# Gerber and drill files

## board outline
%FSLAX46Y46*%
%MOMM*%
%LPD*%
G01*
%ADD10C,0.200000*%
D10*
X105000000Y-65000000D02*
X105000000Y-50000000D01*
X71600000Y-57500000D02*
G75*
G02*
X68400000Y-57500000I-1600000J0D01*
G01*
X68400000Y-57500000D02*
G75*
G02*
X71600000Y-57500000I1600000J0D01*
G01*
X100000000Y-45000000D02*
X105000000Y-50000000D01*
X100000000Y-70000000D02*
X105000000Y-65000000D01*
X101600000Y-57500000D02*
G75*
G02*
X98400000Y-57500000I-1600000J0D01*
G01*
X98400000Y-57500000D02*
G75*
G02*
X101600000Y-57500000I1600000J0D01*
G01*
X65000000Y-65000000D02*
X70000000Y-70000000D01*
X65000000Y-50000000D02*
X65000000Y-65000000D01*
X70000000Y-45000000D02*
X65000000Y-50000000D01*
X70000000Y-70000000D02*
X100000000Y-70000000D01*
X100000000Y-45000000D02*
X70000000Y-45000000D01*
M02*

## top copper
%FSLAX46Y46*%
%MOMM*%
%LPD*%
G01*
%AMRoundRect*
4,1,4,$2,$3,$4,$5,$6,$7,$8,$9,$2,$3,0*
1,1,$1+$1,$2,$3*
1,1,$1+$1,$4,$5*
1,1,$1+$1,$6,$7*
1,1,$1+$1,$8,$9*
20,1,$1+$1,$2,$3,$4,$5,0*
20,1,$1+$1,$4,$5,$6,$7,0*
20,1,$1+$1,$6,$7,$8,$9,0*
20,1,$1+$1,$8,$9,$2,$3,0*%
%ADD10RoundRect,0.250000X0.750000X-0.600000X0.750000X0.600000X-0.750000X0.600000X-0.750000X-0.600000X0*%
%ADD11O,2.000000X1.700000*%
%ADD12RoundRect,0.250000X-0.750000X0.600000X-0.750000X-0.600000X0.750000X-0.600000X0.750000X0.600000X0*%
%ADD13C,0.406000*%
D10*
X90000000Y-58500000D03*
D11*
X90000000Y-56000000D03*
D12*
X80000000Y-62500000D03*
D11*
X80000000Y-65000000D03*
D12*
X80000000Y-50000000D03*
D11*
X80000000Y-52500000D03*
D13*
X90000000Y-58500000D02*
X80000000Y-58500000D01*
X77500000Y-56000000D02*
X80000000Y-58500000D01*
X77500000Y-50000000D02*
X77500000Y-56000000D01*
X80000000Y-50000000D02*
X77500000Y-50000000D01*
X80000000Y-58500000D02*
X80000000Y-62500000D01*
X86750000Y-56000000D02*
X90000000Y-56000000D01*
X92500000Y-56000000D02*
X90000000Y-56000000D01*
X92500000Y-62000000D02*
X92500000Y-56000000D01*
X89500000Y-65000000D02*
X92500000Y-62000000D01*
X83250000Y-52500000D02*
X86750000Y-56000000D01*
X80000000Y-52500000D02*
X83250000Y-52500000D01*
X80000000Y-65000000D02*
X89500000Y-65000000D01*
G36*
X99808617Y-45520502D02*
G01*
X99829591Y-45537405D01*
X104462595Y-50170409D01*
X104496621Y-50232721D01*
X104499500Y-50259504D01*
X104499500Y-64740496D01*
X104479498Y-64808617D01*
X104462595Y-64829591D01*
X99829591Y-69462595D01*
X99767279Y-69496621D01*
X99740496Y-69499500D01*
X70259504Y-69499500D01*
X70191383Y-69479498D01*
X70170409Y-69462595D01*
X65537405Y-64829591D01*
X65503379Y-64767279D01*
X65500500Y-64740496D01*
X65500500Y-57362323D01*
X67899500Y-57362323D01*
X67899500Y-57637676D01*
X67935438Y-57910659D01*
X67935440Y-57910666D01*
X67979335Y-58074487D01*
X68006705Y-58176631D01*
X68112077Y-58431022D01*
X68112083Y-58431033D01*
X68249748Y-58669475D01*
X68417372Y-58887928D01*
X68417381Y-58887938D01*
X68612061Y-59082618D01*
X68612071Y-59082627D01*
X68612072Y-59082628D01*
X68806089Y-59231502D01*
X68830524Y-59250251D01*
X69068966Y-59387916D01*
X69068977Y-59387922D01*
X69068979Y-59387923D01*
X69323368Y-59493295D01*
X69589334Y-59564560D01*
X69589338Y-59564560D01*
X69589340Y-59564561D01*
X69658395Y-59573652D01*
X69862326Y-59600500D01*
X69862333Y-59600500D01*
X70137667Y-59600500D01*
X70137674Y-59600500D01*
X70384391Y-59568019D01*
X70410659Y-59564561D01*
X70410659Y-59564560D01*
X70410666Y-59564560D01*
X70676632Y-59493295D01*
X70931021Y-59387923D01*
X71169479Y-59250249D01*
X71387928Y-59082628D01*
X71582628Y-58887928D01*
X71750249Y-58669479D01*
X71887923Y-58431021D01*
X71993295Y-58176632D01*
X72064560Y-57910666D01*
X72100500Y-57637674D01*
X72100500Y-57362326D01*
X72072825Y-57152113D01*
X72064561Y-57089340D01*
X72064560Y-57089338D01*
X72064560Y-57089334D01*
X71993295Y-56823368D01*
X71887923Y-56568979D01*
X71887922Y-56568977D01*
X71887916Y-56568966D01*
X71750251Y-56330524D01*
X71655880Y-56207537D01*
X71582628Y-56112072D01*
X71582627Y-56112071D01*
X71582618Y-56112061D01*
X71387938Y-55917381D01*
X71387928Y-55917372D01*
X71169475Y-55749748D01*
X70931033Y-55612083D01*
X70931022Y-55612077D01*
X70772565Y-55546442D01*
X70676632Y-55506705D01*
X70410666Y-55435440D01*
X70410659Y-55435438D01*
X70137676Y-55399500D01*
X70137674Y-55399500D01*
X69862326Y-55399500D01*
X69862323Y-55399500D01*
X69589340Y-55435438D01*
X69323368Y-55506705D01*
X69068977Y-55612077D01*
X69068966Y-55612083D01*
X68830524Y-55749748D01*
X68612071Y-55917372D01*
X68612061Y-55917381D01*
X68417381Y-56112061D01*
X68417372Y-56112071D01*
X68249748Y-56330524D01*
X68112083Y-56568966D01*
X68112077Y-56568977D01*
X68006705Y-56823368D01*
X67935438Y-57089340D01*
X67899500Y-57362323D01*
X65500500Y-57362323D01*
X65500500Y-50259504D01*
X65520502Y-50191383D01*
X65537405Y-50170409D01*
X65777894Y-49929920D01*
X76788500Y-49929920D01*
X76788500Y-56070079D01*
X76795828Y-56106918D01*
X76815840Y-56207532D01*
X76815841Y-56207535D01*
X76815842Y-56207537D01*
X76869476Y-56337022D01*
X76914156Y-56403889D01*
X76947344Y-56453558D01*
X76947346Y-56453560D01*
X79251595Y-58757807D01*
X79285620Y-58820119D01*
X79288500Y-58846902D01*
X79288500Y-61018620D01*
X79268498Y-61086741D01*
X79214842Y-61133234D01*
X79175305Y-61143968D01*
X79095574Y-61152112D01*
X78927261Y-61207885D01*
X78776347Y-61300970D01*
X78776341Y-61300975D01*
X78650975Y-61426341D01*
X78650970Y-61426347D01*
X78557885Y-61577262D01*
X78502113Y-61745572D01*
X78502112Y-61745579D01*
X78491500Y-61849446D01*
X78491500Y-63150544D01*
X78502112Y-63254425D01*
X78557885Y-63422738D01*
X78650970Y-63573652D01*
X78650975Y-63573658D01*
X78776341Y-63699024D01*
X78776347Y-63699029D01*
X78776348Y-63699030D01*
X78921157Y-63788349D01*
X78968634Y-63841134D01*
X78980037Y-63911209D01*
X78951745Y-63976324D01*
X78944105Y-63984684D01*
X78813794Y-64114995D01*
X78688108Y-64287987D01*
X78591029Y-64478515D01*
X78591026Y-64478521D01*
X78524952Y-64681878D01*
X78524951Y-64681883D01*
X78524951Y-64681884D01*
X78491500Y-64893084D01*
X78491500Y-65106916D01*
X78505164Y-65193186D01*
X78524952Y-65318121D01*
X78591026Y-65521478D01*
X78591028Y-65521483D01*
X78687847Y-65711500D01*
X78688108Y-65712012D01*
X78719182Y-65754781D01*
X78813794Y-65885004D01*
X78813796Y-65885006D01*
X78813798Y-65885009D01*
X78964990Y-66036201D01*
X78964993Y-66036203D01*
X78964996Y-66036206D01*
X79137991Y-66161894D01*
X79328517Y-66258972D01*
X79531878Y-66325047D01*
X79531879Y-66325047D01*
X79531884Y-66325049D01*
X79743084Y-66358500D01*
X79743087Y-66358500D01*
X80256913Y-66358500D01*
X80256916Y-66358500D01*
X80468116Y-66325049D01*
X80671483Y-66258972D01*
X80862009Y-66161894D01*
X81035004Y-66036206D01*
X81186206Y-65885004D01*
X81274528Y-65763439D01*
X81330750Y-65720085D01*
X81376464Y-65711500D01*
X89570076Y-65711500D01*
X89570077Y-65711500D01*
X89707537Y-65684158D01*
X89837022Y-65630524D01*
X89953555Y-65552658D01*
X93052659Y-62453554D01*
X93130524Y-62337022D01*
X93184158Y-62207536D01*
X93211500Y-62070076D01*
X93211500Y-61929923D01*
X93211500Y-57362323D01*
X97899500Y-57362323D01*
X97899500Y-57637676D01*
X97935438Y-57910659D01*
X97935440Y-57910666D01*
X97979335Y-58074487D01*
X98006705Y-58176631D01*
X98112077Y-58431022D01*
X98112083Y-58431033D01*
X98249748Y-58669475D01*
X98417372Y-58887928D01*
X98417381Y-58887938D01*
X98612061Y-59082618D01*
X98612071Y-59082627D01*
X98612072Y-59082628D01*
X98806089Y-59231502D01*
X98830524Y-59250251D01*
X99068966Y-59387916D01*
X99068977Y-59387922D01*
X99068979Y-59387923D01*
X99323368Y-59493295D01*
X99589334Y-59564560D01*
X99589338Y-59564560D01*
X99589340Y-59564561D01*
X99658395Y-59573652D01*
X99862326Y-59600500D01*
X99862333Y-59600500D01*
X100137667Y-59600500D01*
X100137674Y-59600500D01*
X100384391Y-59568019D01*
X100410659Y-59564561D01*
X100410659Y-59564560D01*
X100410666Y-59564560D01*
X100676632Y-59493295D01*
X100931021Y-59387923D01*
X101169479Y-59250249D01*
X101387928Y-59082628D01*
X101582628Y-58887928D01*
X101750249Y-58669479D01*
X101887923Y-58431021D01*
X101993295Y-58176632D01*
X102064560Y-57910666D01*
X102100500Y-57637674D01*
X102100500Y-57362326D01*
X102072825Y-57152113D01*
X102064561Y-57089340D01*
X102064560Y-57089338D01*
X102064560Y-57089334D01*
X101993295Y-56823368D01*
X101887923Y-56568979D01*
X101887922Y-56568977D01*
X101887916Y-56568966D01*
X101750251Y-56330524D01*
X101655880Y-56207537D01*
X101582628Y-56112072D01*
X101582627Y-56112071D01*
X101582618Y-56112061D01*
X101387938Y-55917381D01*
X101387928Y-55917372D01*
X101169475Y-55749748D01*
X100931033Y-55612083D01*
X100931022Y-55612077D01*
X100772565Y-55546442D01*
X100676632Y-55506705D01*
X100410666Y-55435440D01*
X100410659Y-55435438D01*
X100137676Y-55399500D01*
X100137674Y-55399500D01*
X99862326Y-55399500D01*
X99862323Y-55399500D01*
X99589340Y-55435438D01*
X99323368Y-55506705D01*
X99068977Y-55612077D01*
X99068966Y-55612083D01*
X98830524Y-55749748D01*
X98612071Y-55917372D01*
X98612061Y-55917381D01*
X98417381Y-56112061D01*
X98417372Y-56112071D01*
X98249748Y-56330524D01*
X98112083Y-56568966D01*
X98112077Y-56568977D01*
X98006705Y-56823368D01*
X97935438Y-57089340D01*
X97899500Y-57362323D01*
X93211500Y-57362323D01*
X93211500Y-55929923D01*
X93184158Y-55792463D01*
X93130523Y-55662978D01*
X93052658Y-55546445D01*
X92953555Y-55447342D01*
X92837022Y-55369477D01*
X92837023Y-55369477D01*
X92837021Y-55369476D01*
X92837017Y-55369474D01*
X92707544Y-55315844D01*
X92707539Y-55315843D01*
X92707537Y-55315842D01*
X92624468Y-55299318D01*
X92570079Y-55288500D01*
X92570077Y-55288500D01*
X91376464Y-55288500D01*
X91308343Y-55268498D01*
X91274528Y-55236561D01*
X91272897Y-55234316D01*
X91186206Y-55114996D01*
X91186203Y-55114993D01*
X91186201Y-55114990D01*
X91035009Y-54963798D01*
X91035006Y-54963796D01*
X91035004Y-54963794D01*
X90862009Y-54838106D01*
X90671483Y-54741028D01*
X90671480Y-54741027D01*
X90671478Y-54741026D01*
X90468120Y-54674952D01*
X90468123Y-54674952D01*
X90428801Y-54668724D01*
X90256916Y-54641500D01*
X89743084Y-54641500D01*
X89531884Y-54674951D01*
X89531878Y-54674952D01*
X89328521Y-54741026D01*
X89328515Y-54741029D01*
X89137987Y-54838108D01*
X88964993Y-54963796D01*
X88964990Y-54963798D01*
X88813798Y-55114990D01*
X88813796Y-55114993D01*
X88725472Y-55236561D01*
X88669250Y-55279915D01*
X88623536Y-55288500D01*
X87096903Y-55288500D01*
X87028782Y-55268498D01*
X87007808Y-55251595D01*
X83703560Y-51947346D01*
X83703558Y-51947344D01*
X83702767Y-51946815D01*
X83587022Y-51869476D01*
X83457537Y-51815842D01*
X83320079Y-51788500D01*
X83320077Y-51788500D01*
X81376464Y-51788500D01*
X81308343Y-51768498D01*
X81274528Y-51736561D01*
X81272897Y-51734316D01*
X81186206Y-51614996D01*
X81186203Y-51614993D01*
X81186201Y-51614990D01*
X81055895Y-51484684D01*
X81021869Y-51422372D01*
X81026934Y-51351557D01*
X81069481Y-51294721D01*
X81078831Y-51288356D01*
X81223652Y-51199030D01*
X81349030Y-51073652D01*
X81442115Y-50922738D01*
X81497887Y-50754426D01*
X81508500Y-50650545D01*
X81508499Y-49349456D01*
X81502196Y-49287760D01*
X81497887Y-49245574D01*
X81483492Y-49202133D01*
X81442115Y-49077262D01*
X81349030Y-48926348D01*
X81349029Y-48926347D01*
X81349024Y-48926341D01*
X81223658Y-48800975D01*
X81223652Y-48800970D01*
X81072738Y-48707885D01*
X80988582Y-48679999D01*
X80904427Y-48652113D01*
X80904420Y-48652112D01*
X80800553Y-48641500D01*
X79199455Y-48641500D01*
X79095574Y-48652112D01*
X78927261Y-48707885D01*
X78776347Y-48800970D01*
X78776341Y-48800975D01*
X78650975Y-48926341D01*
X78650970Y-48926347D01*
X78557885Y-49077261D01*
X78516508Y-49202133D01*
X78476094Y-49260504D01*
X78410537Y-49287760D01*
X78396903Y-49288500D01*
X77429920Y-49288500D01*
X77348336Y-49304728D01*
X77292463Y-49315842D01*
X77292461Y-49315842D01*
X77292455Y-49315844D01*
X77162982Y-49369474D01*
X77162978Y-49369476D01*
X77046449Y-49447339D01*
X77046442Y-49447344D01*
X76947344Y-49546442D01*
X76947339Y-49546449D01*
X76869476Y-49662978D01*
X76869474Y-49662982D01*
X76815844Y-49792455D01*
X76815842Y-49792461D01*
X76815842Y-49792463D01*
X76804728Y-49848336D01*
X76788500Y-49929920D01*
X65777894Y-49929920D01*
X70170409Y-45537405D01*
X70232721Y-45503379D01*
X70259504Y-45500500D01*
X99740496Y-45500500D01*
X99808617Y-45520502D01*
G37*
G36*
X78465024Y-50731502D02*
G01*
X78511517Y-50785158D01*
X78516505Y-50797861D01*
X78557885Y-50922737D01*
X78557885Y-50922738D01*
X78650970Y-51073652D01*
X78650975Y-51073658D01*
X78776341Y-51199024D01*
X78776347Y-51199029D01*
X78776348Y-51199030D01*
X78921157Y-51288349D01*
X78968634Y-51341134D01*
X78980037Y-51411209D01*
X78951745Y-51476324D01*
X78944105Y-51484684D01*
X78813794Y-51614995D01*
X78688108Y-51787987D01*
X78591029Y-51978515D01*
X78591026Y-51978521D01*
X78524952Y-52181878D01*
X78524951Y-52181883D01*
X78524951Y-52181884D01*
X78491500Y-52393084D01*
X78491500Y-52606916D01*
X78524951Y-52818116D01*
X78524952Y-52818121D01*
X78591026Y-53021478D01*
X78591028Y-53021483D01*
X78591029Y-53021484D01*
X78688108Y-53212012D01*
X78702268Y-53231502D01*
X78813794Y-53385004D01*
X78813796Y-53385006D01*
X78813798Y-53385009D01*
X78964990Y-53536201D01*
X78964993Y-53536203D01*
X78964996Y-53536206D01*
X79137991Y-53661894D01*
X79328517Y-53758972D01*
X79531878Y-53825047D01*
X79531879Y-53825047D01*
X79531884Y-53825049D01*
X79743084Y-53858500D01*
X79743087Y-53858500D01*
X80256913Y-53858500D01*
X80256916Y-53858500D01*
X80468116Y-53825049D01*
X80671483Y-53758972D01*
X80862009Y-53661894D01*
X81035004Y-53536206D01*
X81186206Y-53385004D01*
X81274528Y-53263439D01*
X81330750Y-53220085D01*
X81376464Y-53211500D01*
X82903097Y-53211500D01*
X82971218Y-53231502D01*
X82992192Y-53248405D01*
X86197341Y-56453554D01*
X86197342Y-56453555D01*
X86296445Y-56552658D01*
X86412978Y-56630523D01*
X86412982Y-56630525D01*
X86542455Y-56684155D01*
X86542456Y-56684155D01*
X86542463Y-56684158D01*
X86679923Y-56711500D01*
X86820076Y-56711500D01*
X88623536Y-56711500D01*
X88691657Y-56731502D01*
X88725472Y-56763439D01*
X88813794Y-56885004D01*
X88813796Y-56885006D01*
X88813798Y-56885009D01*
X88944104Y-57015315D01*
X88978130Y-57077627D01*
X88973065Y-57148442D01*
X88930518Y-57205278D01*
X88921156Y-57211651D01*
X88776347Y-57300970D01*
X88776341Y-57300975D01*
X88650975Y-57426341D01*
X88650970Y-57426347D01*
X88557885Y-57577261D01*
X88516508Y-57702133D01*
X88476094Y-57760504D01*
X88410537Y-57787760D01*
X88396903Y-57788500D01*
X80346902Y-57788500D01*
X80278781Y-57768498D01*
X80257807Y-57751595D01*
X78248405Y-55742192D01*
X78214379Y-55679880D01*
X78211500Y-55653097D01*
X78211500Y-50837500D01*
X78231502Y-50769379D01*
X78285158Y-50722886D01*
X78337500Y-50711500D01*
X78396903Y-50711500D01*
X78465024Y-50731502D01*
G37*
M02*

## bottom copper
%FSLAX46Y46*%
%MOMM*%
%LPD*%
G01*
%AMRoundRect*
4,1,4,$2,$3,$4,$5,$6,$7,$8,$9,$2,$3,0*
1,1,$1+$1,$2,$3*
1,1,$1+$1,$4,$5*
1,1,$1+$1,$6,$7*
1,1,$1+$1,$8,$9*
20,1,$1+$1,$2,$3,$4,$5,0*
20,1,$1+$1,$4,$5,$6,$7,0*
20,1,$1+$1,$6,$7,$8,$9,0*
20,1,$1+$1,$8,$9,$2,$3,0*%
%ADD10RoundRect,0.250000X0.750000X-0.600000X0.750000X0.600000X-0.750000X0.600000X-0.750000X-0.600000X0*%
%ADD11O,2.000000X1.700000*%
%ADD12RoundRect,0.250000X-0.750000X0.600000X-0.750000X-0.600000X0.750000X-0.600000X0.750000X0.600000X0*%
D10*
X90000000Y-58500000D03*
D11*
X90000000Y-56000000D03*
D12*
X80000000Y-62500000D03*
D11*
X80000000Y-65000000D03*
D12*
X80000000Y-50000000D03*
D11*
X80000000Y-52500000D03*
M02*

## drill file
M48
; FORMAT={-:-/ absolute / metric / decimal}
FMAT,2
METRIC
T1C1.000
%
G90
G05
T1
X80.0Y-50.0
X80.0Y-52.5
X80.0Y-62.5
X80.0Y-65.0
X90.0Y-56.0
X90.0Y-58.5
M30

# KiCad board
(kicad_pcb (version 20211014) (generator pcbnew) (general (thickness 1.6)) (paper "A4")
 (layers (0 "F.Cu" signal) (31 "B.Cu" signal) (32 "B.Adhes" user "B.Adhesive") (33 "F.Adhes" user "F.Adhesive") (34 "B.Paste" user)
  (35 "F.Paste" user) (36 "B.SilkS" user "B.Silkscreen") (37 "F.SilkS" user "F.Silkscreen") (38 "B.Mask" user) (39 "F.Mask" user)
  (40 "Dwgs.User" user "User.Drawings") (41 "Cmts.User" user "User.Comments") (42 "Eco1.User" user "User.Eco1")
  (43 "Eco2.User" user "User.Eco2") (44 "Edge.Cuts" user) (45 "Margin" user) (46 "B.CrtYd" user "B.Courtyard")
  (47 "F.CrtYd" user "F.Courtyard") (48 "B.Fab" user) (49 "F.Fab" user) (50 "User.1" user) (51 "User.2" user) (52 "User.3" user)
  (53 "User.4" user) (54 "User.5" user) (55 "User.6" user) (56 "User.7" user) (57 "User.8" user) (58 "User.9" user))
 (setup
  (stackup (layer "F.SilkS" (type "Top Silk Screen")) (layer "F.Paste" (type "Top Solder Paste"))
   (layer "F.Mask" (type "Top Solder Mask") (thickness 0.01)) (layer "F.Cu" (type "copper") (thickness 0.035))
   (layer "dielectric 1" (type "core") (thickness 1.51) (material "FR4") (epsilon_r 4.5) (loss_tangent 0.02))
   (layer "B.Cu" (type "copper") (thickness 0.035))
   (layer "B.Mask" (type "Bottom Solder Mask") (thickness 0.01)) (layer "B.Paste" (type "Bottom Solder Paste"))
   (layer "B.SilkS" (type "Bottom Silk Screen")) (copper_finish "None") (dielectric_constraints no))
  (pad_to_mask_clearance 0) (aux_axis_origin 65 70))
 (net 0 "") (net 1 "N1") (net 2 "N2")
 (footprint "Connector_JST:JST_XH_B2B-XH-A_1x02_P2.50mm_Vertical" (layer "F.Cu") (at 90 58.5 90)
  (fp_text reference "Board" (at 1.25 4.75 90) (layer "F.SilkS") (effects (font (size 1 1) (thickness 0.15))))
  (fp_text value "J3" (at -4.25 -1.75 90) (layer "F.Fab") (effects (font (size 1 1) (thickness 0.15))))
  (pad "1" thru_hole roundrect (at 0 0 90) (size 1.7 2) (drill 1) (layers *.Cu *.Mask) (roundrect_rratio 0.1470588235) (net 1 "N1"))
  (pad "2" thru_hole oval (at 2.5 0 90) (size 1.7 2) (drill 1) (layers *.Cu *.Mask) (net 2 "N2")))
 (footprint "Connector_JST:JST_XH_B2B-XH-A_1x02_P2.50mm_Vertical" (layer "F.Cu") (at 80 62.5 -90)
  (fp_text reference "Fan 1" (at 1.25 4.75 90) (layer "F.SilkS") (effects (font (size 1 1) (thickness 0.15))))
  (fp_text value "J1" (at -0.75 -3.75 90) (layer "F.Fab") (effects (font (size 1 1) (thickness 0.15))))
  (pad "1" thru_hole roundrect (at 0 0 270) (size 1.7 2) (drill 1) (layers *.Cu *.Mask) (roundrect_rratio 0.1470588235) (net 1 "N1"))
  (pad "2" thru_hole oval (at 2.5 0 270) (size 1.7 2) (drill 1) (layers *.Cu *.Mask) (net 2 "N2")))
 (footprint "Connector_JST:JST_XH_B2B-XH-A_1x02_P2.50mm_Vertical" (layer "F.Cu") (at 80 50 -90)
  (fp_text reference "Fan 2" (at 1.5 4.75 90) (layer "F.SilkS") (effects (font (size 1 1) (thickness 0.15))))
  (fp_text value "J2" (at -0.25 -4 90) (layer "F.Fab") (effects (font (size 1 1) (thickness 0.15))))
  (pad "1" thru_hole roundrect (at 0 0 270) (size 1.7 2) (drill 1) (layers *.Cu *.Mask) (roundrect_rratio 0.1470588235) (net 1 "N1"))
  (pad "2" thru_hole oval (at 2.5 0 270) (size 1.7 2) (drill 1) (layers *.Cu *.Mask) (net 2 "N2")))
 (gr_line (start 105 65) (end 105 50) (layer "Edge.Cuts") (width 0.2))
 (gr_circle (center 70 57.5) (end 71.6 57.5) (layer "Edge.Cuts") (width 0.2) (fill none))
 (gr_line (start 100 45) (end 105 50) (layer "Edge.Cuts") (width 0.2))
 (gr_line (start 100 70) (end 105 65) (layer "Edge.Cuts") (width 0.2))
 (gr_circle (center 100 57.5) (end 101.6 57.5) (layer "Edge.Cuts") (width 0.2) (fill none))
 (gr_line (start 65 65) (end 70 70) (layer "Edge.Cuts") (width 0.2))
 (gr_line (start 65 50) (end 65 65) (layer "Edge.Cuts") (width 0.2))
 (gr_line (start 70 45) (end 65 50) (layer "Edge.Cuts") (width 0.2))
 (gr_line (start 70 70) (end 100 70) (layer "Edge.Cuts") (width 0.2))
 (gr_line (start 100 45) (end 70 45) (layer "Edge.Cuts") (width 0.2))
 (segment (start 90 58.5) (end 80 58.5) (width 0.406) (layer "F.Cu") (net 1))
 (segment (start 77.5 56) (end 80 58.5) (width 0.406) (layer "F.Cu") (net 1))
 (segment (start 77.5 50) (end 77.5 56) (width 0.406) (layer "F.Cu") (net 1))
 (segment (start 80 50) (end 77.5 50) (width 0.406) (layer "F.Cu") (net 1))
 (segment (start 80 58.5) (end 80 62.5) (width 0.406) (layer "F.Cu") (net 1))
 (segment (start 86.75 56) (end 90 56) (width 0.406) (layer "F.Cu") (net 2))
 (segment (start 92.5 56) (end 90 56) (width 0.406) (layer "F.Cu") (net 2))
 (segment (start 92.5 62) (end 92.5 56) (width 0.406) (layer "F.Cu") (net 2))
 (segment (start 89.5 65) (end 92.5 62) (width 0.406) (layer "F.Cu") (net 2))
 (segment (start 83.25 52.5) (end 86.75 56) (width 0.406) (layer "F.Cu") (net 2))
 (segment (start 80 52.5) (end 83.25 52.5) (width 0.406) (layer "F.Cu") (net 2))
 (segment (start 80 65) (end 89.5 65) (width 0.406) (layer "F.Cu") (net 2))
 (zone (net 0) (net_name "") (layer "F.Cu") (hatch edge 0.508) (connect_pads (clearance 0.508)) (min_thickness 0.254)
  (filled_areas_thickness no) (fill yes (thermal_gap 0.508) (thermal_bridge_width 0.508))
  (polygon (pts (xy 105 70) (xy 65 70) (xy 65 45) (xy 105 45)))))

